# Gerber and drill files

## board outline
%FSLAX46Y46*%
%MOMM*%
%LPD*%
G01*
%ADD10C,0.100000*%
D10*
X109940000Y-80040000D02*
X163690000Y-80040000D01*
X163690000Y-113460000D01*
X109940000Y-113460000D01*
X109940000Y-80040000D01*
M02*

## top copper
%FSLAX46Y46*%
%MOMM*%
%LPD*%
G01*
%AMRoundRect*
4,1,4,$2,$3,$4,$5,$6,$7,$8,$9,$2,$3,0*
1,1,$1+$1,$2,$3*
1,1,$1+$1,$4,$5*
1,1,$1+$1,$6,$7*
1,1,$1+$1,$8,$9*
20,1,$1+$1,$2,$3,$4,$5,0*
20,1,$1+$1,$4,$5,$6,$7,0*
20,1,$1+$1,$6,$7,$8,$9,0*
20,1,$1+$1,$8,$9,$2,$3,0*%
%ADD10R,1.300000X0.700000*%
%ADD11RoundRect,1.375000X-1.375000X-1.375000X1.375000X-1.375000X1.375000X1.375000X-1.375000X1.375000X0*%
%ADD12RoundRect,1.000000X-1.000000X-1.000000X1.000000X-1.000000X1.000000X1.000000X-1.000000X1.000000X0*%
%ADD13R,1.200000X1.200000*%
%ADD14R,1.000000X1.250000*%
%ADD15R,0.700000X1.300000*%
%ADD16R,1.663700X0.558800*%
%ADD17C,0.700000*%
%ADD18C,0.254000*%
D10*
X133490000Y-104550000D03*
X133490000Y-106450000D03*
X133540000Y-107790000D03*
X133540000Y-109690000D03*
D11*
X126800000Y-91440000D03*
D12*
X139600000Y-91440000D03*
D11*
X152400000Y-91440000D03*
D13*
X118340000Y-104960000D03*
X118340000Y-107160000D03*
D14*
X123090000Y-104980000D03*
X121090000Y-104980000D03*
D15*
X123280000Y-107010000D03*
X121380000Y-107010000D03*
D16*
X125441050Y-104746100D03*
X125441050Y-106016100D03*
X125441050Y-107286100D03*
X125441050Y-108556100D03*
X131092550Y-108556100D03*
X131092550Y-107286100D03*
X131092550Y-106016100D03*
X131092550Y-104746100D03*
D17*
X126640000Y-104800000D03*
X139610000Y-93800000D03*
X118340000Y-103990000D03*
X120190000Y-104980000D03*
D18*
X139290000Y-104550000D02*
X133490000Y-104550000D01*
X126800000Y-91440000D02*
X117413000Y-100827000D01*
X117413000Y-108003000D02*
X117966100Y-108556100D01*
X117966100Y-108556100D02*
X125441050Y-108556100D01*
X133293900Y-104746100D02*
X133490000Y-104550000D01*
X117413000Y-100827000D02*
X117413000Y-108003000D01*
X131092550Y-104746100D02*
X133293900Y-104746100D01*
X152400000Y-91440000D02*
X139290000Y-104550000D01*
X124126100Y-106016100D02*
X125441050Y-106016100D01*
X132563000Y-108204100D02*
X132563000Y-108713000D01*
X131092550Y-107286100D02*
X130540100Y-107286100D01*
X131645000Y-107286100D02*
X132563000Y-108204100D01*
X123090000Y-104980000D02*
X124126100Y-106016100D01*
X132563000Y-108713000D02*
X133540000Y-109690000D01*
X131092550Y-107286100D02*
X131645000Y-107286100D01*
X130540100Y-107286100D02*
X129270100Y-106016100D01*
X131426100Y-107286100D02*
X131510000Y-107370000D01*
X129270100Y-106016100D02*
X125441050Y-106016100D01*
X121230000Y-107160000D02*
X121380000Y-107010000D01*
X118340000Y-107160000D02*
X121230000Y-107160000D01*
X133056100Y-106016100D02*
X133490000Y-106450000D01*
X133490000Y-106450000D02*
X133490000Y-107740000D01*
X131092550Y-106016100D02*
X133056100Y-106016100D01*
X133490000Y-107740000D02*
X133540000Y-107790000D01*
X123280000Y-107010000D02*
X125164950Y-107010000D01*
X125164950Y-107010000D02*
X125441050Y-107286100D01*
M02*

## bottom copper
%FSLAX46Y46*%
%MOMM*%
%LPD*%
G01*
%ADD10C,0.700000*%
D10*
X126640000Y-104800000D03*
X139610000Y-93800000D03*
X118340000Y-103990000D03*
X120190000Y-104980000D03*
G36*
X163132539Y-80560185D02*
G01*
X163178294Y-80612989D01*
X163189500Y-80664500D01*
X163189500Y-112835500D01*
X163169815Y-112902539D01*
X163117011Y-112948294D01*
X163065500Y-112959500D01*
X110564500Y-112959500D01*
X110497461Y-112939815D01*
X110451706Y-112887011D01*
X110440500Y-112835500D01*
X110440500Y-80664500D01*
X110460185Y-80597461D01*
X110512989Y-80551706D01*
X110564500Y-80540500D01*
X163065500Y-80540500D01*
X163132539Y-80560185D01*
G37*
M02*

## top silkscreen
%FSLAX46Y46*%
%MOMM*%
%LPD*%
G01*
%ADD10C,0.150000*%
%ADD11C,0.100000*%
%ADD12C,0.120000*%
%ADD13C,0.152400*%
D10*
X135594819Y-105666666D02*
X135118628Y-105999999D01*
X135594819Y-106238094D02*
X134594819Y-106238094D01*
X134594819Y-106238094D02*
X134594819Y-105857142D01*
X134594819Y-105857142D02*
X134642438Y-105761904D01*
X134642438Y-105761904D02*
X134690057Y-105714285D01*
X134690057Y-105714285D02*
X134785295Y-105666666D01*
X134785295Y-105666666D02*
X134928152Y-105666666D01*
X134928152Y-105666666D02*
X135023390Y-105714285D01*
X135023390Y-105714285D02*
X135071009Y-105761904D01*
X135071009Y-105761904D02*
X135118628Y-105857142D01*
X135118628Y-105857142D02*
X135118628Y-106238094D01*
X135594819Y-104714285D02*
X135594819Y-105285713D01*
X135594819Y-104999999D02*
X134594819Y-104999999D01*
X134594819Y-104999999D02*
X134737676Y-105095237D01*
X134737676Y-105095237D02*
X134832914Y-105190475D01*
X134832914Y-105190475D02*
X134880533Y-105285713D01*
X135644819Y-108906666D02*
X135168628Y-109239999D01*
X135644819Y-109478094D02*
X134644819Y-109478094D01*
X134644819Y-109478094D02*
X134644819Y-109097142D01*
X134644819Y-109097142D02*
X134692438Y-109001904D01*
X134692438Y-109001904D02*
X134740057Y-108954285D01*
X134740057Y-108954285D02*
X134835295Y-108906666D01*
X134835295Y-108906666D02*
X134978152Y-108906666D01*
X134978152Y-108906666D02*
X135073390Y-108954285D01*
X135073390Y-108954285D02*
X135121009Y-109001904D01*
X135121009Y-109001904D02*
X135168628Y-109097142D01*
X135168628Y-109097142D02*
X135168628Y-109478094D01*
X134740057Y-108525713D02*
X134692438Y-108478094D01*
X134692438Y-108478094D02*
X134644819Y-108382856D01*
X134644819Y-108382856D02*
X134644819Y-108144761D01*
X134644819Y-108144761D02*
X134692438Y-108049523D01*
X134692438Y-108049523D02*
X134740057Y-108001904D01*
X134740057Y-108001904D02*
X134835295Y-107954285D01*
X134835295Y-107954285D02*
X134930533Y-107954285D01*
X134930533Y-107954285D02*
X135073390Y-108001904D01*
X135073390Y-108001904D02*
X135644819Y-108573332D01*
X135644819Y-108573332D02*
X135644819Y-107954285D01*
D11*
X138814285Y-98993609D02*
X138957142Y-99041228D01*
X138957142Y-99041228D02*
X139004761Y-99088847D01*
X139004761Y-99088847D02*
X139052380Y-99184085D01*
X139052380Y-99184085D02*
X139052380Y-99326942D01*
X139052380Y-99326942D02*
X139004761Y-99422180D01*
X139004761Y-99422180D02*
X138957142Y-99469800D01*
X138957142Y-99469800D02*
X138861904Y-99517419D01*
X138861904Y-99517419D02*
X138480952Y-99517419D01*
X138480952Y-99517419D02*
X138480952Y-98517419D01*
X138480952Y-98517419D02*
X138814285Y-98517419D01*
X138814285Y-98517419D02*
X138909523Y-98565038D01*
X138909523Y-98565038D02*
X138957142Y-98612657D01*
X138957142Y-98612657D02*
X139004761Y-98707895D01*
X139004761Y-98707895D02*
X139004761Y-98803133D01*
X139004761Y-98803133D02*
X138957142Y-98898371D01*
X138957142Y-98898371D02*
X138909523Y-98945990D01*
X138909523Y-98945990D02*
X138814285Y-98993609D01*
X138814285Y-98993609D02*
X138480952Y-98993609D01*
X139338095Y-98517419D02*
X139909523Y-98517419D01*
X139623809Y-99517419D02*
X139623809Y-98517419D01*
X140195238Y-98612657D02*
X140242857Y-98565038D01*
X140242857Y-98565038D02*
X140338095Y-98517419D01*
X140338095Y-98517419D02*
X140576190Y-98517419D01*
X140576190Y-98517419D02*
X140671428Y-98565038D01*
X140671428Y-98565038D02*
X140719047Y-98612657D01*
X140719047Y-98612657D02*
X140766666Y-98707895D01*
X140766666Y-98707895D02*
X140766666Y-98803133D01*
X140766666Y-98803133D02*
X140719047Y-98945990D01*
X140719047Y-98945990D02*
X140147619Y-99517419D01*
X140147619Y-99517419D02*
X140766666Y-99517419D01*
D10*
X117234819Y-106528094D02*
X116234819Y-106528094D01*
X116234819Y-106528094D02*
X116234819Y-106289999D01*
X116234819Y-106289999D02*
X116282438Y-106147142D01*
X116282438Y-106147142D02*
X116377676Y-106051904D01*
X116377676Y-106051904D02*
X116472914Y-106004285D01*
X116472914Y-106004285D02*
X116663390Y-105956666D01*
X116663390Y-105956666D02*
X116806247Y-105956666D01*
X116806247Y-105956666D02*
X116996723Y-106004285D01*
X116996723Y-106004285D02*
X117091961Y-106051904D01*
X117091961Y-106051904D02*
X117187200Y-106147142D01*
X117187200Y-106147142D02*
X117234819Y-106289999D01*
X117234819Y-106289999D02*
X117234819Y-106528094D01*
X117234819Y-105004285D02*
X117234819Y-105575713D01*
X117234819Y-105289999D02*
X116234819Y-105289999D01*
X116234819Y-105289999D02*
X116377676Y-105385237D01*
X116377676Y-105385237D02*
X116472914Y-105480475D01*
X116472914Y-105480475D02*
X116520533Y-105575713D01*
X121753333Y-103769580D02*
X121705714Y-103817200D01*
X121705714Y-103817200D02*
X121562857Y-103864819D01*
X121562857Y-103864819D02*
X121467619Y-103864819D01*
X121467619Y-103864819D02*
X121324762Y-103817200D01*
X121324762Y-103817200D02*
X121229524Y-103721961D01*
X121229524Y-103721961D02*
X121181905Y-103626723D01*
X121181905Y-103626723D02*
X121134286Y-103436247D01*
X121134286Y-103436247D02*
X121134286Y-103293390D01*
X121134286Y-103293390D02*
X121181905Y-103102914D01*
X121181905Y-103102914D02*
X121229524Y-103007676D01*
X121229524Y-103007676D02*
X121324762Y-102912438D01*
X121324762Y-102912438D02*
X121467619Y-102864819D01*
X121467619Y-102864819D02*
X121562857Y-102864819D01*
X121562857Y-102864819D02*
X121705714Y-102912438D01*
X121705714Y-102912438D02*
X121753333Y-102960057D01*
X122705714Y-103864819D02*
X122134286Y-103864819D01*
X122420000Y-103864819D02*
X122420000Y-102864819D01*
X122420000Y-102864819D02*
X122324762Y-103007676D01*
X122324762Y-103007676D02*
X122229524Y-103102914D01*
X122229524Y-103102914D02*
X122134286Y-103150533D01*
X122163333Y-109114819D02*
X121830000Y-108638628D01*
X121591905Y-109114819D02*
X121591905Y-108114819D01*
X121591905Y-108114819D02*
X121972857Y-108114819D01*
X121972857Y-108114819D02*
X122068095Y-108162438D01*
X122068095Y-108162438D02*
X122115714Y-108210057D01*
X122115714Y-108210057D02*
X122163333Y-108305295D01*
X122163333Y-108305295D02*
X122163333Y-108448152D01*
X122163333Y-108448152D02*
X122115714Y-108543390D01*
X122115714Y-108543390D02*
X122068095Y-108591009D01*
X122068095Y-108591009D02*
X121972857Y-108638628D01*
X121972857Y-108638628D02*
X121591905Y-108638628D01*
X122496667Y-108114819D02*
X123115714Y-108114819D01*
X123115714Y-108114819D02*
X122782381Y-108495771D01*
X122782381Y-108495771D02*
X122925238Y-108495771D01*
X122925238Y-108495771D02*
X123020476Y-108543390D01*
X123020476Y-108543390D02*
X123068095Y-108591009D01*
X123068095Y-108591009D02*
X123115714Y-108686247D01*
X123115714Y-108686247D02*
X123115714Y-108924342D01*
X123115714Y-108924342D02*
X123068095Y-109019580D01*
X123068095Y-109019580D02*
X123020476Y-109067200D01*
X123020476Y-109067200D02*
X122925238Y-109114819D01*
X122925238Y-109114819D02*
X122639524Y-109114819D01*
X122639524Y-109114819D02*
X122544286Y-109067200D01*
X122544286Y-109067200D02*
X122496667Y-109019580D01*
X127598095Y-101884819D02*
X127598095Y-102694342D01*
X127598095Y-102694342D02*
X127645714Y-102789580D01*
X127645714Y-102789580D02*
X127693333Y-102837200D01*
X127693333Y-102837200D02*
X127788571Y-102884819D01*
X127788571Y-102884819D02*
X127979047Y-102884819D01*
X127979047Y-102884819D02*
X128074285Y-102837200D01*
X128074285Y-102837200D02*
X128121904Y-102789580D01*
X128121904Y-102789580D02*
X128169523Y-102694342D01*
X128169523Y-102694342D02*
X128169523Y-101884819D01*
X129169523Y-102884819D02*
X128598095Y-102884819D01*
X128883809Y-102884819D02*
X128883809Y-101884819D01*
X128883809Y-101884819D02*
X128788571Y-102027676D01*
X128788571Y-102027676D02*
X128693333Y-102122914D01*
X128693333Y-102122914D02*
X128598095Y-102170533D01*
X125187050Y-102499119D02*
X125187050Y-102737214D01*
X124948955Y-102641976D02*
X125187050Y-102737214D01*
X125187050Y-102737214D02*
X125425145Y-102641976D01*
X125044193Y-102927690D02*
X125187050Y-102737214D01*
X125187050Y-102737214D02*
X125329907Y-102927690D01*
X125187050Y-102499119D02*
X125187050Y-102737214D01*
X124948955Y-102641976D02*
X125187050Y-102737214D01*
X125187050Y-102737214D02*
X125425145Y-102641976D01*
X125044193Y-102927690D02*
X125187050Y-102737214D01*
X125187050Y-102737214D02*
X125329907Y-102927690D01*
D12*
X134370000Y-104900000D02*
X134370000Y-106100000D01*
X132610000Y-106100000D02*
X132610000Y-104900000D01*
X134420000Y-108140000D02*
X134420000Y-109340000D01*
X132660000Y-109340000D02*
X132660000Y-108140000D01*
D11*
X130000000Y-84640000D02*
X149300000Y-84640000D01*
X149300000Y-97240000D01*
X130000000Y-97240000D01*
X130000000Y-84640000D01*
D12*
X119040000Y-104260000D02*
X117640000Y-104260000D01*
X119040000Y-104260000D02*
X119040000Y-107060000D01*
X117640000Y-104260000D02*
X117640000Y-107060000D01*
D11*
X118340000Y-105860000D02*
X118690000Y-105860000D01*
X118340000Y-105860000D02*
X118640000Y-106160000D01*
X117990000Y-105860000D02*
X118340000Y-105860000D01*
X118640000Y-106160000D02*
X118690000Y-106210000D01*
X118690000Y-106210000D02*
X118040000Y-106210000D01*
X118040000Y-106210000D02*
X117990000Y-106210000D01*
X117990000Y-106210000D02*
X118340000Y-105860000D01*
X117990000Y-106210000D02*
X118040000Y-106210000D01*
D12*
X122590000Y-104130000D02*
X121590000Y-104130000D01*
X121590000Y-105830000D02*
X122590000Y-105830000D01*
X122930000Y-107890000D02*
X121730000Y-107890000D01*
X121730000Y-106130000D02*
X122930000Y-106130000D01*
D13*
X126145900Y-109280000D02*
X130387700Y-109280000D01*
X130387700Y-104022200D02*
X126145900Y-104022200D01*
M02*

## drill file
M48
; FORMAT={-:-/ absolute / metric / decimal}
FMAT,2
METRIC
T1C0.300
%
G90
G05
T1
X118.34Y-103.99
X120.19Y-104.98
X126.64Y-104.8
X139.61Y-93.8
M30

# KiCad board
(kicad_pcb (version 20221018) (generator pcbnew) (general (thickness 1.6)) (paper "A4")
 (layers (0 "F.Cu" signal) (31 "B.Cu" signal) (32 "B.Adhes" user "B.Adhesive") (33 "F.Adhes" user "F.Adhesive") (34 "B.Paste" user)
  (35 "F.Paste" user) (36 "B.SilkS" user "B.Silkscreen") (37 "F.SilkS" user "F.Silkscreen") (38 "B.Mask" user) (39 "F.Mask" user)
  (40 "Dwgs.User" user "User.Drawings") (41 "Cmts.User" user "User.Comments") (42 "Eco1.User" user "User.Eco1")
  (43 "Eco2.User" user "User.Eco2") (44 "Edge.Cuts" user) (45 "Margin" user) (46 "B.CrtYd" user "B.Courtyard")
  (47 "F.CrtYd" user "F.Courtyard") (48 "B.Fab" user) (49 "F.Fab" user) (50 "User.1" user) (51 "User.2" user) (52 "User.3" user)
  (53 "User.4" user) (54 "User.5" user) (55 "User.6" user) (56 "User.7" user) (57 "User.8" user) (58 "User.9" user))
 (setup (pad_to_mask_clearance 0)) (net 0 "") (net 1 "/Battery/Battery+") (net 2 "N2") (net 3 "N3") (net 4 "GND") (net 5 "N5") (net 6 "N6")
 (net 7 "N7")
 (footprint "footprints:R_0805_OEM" (layer "F.Cu") (at 133.49 105.5 -90)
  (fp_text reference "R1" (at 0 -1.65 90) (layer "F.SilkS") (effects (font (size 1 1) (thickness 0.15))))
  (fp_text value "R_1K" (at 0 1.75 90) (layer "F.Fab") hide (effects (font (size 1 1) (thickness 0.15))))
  (fp_line (start -0.6 -0.88) (end 0.6 -0.88) (stroke (width 0.12) (type solid)) (layer "F.SilkS"))
  (fp_line (start 0.6 0.88) (end -0.6 0.88) (stroke (width 0.12) (type solid)) (layer "F.SilkS"))
  (pad "1" smd rect (at -0.95 0 270) (size 0.7 1.3) (layers "F.Cu" "F.Paste" "F.Mask") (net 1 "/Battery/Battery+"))
  (pad "2" smd rect (at 0.95 0 270) (size 0.7 1.3) (layers "F.Cu" "F.Paste" "F.Mask") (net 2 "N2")))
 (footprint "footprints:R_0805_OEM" (layer "F.Cu") (at 133.54 108.74 -90)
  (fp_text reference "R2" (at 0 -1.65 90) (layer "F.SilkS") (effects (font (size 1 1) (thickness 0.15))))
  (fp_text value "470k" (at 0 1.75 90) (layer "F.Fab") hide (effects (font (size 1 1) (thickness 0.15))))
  (fp_line (start -0.6 -0.88) (end 0.6 -0.88) (stroke (width 0.12) (type solid)) (layer "F.SilkS"))
  (fp_line (start 0.6 0.88) (end -0.6 0.88) (stroke (width 0.12) (type solid)) (layer "F.SilkS"))
  (pad "1" smd rect (at -0.95 0 270) (size 0.7 1.3) (layers "F.Cu" "F.Paste" "F.Mask") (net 2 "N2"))
  (pad "2" smd rect (at 0.95 0 270) (size 0.7 1.3) (layers "F.Cu" "F.Paste" "F.Mask") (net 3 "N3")))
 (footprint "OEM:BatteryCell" (layer "F.Cu") (at 139.6 91.44)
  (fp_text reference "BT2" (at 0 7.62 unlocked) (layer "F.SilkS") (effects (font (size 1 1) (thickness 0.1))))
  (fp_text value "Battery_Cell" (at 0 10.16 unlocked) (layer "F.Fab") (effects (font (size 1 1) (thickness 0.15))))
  (fp_rect (start -9.6 -6.8) (end 9.7 5.8) (stroke (width 0.1) (type default)) (fill none) (layer "F.SilkS"))
  (pad "1" smd roundrect (at -12.8 0) (size 5.5 5.5) (layers "F.Cu" "F.Paste" "F.Mask") (roundrect_rratio 0.25) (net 1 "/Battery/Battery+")
   (thermal_bridge_angle 45))
  (pad "2" smd roundrect (at 0 0) (size 4 4) (layers "F.Cu" "F.Paste" "F.Mask") (roundrect_rratio 0.25) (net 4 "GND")
   (thermal_bridge_angle 45))
  (pad "3" smd roundrect (at 12.8 0) (size 5.5 5.5) (layers "F.Cu" "F.Paste" "F.Mask") (roundrect_rratio 0.25) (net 1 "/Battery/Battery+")
   (thermal_bridge_angle 45)))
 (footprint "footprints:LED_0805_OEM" (layer "F.Cu") (at 118.34 106.06 -90)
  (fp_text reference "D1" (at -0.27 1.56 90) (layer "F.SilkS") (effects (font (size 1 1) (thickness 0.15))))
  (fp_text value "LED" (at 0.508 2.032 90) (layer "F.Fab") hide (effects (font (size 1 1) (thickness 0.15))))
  (fp_line (start -1.8 -0.7) (end -1.8 0.7) (stroke (width 0.12) (type solid)) (layer "F.SilkS"))
  (fp_line (start -1.8 -0.7) (end 1 -0.7) (stroke (width 0.12) (type solid)) (layer "F.SilkS"))
  (fp_line (start -1.8 0.7) (end 1 0.7) (stroke (width 0.12) (type solid)) (layer "F.SilkS"))
  (fp_line (start -0.2 0) (end -0.2 -0.35) (stroke (width 0.1) (type solid)) (layer "F.SilkS"))
  (fp_line (start -0.2 0) (end 0.1 -0.3) (stroke (width 0.1) (type solid)) (layer "F.SilkS"))
  (fp_line (start -0.2 0.35) (end -0.2 0) (stroke (width 0.1) (type solid)) (layer "F.SilkS"))
  (fp_line (start 0.1 -0.3) (end 0.15 -0.35) (stroke (width 0.1) (type solid)) (layer "F.SilkS"))
  (fp_line (start 0.15 -0.35) (end 0.15 0.3) (stroke (width 0.1) (type solid)) (layer "F.SilkS"))
  (fp_line (start 0.15 0.3) (end 0.15 0.35) (stroke (width 0.1) (type solid)) (layer "F.SilkS"))
  (fp_line (start 0.15 0.35) (end -0.2 0) (stroke (width 0.1) (type solid)) (layer "F.SilkS"))
  (fp_line (start 0.15 0.35) (end 0.15 0.3) (stroke (width 0.1) (type solid)) (layer "F.SilkS"))
  (pad "1" smd rect (at -1.1 0 90) (size 1.2 1.2) (layers "F.Cu" "F.Paste" "F.Mask") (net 4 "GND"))
  (pad "2" smd rect (at 1.1 0 90) (size 1.2 1.2) (layers "F.Cu" "F.Paste" "F.Mask") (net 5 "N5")))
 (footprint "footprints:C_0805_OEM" (layer "F.Cu") (at 122.09 104.98 180)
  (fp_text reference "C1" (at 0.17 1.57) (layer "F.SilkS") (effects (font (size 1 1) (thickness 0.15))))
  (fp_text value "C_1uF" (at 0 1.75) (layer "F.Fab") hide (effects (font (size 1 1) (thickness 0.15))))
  (fp_line (start -0.5 0.85) (end 0.5 0.85) (stroke (width 0.12) (type solid)) (layer "F.SilkS"))
  (fp_line (start 0.5 -0.85) (end -0.5 -0.85) (stroke (width 0.12) (type solid)) (layer "F.SilkS"))
  (pad "1" smd rect (at -1 0 180) (size 1 1.25) (layers "F.Cu" "F.Paste" "F.Mask") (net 3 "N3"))
  (pad "2" smd rect (at 1 0 180) (size 1 1.25) (layers "F.Cu" "F.Paste" "F.Mask") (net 4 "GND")))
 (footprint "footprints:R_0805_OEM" (layer "F.Cu") (at 122.33 107.01 180)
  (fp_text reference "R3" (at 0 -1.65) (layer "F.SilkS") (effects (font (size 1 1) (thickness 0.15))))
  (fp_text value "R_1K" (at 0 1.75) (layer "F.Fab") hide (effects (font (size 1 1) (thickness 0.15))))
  (fp_line (start -0.6 -0.88) (end 0.6 -0.88) (stroke (width 0.12) (type solid)) (layer "F.SilkS"))
  (fp_line (start 0.6 0.88) (end -0.6 0.88) (stroke (width 0.12) (type solid)) (layer "F.SilkS"))
  (pad "1" smd rect (at -0.95 0 180) (size 0.7 1.3) (layers "F.Cu" "F.Paste" "F.Mask") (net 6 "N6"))
  (pad "2" smd rect (at 0.95 0 180) (size 0.7 1.3) (layers "F.Cu" "F.Paste" "F.Mask") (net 5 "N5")))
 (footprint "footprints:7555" (layer "F.Cu") (at 128.2668 106.6511)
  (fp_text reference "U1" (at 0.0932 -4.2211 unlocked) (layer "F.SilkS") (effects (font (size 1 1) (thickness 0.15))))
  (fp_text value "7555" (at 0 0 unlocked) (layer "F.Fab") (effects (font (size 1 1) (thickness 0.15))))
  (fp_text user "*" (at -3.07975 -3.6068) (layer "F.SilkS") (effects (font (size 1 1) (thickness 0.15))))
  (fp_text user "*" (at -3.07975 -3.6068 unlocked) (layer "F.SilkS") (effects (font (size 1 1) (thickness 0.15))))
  (fp_line (start -2.1209 2.6289) (end 2.1209 2.6289) (stroke (width 0.1524) (type solid)) (layer "F.SilkS"))
  (fp_line (start 2.1209 -2.6289) (end -2.1209 -2.6289) (stroke (width 0.1524) (type solid)) (layer "F.SilkS"))
  (pad "1" smd rect (at -2.82575 -1.905) (size 1.6637 0.5588) (layers "F.Cu" "F.Paste" "F.Mask") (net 4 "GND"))
  (pad "2" smd rect (at -2.82575 -0.635) (size 1.6637 0.5588) (layers "F.Cu" "F.Paste" "F.Mask") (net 3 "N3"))
  (pad "3" smd rect (at -2.82575 0.635) (size 1.6637 0.5588) (layers "F.Cu" "F.Paste" "F.Mask") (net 6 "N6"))
  (pad "4" smd rect (at -2.82575 1.905) (size 1.6637 0.5588) (layers "F.Cu" "F.Paste" "F.Mask") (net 1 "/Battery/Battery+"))
  (pad "5" smd rect (at 2.82575 1.905) (size 1.6637 0.5588) (layers "F.Cu" "F.Paste" "F.Mask") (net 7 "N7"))
  (pad "6" smd rect (at 2.82575 0.635) (size 1.6637 0.5588) (layers "F.Cu" "F.Paste" "F.Mask") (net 3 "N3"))
  (pad "7" smd rect (at 2.82575 -0.635) (size 1.6637 0.5588) (layers "F.Cu" "F.Paste" "F.Mask") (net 2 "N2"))
  (pad "8" smd rect (at 2.82575 -1.905) (size 1.6637 0.5588) (layers "F.Cu" "F.Paste" "F.Mask") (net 1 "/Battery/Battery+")))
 (gr_rect (start 109.94 80.04) (end 163.69 113.46) (stroke (width 0.1) (type default)) (fill none) (layer "Edge.Cuts"))
 (segment (start 139.29 104.55) (end 133.49 104.55) (width 0.254) (layer "F.Cu") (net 1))
 (segment (start 126.8 91.44) (end 117.413 100.827) (width 0.254) (layer "F.Cu") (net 1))
 (segment (start 117.413 108.003) (end 117.9661 108.5561) (width 0.254) (layer "F.Cu") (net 1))
 (segment (start 117.9661 108.5561) (end 125.44105 108.5561) (width 0.254) (layer "F.Cu") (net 1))
 (segment (start 133.2939 104.7461) (end 133.49 104.55) (width 0.254) (layer "F.Cu") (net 1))
 (segment (start 117.413 100.827) (end 117.413 108.003) (width 0.254) (layer "F.Cu") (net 1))
 (segment (start 131.09255 104.7461) (end 133.2939 104.7461) (width 0.254) (layer "F.Cu") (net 1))
 (segment (start 152.4 91.44) (end 139.29 104.55) (width 0.254) (layer "F.Cu") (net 1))
 (via (at 126.64 104.8) (size 0.7) (drill 0.3) (layers "F.Cu" "B.Cu") (free) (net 4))
 (via (at 139.61 93.8) (size 0.7) (drill 0.3) (layers "F.Cu" "B.Cu") (free) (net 4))
 (via (at 118.34 103.99) (size 0.7) (drill 0.3) (layers "F.Cu" "B.Cu") (free) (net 4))
 (via (at 120.19 104.98) (size 0.7) (drill 0.3) (layers "F.Cu" "B.Cu") (free) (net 4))
 (segment (start 124.1261 106.0161) (end 125.44105 106.0161) (width 0.254) (layer "F.Cu") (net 3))
 (segment (start 132.563 108.2041) (end 132.563 108.713) (width 0.254) (layer "F.Cu") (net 3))
 (segment (start 131.09255 107.2861) (end 130.5401 107.2861) (width 0.254) (layer "F.Cu") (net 3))
 (segment (start 131.645 107.2861) (end 132.563 108.2041) (width 0.254) (layer "F.Cu") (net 3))
 (segment (start 123.09 104.98) (end 124.1261 106.0161) (width 0.254) (layer "F.Cu") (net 3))
 (segment (start 132.563 108.713) (end 133.54 109.69) (width 0.254) (layer "F.Cu") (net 3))
 (segment (start 131.09255 107.2861) (end 131.645 107.2861) (width 0.254) (layer "F.Cu") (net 3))
 (segment (start 130.5401 107.2861) (end 129.2701 106.0161) (width 0.254) (layer "F.Cu") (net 3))
 (segment (start 131.4261 107.2861) (end 131.51 107.37) (width 0.254) (layer "F.Cu") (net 3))
 (segment (start 129.2701 106.0161) (end 125.44105 106.0161) (width 0.254) (layer "F.Cu") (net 3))
 (segment (start 121.23 107.16) (end 121.38 107.01) (width 0.254) (layer "F.Cu") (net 5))
 (segment (start 118.34 107.16) (end 121.23 107.16) (width 0.254) (layer "F.Cu") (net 5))
 (segment (start 133.0561 106.0161) (end 133.49 106.45) (width 0.254) (layer "F.Cu") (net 2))
 (segment (start 133.49 106.45) (end 133.49 107.74) (width 0.254) (layer "F.Cu") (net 2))
 (segment (start 131.09255 106.0161) (end 133.0561 106.0161) (width 0.254) (layer "F.Cu") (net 2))
 (segment (start 133.49 107.74) (end 133.54 107.79) (width 0.254) (layer "F.Cu") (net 2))
 (segment (start 123.28 107.01) (end 125.16495 107.01) (width 0.254) (layer "F.Cu") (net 6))
 (segment (start 125.16495 107.01) (end 125.44105 107.2861) (width 0.254) (layer "F.Cu") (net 6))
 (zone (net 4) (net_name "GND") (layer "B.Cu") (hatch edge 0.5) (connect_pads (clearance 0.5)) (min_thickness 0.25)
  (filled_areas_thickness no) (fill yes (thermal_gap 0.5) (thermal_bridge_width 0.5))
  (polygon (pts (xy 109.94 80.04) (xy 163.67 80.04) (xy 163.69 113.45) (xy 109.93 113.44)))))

